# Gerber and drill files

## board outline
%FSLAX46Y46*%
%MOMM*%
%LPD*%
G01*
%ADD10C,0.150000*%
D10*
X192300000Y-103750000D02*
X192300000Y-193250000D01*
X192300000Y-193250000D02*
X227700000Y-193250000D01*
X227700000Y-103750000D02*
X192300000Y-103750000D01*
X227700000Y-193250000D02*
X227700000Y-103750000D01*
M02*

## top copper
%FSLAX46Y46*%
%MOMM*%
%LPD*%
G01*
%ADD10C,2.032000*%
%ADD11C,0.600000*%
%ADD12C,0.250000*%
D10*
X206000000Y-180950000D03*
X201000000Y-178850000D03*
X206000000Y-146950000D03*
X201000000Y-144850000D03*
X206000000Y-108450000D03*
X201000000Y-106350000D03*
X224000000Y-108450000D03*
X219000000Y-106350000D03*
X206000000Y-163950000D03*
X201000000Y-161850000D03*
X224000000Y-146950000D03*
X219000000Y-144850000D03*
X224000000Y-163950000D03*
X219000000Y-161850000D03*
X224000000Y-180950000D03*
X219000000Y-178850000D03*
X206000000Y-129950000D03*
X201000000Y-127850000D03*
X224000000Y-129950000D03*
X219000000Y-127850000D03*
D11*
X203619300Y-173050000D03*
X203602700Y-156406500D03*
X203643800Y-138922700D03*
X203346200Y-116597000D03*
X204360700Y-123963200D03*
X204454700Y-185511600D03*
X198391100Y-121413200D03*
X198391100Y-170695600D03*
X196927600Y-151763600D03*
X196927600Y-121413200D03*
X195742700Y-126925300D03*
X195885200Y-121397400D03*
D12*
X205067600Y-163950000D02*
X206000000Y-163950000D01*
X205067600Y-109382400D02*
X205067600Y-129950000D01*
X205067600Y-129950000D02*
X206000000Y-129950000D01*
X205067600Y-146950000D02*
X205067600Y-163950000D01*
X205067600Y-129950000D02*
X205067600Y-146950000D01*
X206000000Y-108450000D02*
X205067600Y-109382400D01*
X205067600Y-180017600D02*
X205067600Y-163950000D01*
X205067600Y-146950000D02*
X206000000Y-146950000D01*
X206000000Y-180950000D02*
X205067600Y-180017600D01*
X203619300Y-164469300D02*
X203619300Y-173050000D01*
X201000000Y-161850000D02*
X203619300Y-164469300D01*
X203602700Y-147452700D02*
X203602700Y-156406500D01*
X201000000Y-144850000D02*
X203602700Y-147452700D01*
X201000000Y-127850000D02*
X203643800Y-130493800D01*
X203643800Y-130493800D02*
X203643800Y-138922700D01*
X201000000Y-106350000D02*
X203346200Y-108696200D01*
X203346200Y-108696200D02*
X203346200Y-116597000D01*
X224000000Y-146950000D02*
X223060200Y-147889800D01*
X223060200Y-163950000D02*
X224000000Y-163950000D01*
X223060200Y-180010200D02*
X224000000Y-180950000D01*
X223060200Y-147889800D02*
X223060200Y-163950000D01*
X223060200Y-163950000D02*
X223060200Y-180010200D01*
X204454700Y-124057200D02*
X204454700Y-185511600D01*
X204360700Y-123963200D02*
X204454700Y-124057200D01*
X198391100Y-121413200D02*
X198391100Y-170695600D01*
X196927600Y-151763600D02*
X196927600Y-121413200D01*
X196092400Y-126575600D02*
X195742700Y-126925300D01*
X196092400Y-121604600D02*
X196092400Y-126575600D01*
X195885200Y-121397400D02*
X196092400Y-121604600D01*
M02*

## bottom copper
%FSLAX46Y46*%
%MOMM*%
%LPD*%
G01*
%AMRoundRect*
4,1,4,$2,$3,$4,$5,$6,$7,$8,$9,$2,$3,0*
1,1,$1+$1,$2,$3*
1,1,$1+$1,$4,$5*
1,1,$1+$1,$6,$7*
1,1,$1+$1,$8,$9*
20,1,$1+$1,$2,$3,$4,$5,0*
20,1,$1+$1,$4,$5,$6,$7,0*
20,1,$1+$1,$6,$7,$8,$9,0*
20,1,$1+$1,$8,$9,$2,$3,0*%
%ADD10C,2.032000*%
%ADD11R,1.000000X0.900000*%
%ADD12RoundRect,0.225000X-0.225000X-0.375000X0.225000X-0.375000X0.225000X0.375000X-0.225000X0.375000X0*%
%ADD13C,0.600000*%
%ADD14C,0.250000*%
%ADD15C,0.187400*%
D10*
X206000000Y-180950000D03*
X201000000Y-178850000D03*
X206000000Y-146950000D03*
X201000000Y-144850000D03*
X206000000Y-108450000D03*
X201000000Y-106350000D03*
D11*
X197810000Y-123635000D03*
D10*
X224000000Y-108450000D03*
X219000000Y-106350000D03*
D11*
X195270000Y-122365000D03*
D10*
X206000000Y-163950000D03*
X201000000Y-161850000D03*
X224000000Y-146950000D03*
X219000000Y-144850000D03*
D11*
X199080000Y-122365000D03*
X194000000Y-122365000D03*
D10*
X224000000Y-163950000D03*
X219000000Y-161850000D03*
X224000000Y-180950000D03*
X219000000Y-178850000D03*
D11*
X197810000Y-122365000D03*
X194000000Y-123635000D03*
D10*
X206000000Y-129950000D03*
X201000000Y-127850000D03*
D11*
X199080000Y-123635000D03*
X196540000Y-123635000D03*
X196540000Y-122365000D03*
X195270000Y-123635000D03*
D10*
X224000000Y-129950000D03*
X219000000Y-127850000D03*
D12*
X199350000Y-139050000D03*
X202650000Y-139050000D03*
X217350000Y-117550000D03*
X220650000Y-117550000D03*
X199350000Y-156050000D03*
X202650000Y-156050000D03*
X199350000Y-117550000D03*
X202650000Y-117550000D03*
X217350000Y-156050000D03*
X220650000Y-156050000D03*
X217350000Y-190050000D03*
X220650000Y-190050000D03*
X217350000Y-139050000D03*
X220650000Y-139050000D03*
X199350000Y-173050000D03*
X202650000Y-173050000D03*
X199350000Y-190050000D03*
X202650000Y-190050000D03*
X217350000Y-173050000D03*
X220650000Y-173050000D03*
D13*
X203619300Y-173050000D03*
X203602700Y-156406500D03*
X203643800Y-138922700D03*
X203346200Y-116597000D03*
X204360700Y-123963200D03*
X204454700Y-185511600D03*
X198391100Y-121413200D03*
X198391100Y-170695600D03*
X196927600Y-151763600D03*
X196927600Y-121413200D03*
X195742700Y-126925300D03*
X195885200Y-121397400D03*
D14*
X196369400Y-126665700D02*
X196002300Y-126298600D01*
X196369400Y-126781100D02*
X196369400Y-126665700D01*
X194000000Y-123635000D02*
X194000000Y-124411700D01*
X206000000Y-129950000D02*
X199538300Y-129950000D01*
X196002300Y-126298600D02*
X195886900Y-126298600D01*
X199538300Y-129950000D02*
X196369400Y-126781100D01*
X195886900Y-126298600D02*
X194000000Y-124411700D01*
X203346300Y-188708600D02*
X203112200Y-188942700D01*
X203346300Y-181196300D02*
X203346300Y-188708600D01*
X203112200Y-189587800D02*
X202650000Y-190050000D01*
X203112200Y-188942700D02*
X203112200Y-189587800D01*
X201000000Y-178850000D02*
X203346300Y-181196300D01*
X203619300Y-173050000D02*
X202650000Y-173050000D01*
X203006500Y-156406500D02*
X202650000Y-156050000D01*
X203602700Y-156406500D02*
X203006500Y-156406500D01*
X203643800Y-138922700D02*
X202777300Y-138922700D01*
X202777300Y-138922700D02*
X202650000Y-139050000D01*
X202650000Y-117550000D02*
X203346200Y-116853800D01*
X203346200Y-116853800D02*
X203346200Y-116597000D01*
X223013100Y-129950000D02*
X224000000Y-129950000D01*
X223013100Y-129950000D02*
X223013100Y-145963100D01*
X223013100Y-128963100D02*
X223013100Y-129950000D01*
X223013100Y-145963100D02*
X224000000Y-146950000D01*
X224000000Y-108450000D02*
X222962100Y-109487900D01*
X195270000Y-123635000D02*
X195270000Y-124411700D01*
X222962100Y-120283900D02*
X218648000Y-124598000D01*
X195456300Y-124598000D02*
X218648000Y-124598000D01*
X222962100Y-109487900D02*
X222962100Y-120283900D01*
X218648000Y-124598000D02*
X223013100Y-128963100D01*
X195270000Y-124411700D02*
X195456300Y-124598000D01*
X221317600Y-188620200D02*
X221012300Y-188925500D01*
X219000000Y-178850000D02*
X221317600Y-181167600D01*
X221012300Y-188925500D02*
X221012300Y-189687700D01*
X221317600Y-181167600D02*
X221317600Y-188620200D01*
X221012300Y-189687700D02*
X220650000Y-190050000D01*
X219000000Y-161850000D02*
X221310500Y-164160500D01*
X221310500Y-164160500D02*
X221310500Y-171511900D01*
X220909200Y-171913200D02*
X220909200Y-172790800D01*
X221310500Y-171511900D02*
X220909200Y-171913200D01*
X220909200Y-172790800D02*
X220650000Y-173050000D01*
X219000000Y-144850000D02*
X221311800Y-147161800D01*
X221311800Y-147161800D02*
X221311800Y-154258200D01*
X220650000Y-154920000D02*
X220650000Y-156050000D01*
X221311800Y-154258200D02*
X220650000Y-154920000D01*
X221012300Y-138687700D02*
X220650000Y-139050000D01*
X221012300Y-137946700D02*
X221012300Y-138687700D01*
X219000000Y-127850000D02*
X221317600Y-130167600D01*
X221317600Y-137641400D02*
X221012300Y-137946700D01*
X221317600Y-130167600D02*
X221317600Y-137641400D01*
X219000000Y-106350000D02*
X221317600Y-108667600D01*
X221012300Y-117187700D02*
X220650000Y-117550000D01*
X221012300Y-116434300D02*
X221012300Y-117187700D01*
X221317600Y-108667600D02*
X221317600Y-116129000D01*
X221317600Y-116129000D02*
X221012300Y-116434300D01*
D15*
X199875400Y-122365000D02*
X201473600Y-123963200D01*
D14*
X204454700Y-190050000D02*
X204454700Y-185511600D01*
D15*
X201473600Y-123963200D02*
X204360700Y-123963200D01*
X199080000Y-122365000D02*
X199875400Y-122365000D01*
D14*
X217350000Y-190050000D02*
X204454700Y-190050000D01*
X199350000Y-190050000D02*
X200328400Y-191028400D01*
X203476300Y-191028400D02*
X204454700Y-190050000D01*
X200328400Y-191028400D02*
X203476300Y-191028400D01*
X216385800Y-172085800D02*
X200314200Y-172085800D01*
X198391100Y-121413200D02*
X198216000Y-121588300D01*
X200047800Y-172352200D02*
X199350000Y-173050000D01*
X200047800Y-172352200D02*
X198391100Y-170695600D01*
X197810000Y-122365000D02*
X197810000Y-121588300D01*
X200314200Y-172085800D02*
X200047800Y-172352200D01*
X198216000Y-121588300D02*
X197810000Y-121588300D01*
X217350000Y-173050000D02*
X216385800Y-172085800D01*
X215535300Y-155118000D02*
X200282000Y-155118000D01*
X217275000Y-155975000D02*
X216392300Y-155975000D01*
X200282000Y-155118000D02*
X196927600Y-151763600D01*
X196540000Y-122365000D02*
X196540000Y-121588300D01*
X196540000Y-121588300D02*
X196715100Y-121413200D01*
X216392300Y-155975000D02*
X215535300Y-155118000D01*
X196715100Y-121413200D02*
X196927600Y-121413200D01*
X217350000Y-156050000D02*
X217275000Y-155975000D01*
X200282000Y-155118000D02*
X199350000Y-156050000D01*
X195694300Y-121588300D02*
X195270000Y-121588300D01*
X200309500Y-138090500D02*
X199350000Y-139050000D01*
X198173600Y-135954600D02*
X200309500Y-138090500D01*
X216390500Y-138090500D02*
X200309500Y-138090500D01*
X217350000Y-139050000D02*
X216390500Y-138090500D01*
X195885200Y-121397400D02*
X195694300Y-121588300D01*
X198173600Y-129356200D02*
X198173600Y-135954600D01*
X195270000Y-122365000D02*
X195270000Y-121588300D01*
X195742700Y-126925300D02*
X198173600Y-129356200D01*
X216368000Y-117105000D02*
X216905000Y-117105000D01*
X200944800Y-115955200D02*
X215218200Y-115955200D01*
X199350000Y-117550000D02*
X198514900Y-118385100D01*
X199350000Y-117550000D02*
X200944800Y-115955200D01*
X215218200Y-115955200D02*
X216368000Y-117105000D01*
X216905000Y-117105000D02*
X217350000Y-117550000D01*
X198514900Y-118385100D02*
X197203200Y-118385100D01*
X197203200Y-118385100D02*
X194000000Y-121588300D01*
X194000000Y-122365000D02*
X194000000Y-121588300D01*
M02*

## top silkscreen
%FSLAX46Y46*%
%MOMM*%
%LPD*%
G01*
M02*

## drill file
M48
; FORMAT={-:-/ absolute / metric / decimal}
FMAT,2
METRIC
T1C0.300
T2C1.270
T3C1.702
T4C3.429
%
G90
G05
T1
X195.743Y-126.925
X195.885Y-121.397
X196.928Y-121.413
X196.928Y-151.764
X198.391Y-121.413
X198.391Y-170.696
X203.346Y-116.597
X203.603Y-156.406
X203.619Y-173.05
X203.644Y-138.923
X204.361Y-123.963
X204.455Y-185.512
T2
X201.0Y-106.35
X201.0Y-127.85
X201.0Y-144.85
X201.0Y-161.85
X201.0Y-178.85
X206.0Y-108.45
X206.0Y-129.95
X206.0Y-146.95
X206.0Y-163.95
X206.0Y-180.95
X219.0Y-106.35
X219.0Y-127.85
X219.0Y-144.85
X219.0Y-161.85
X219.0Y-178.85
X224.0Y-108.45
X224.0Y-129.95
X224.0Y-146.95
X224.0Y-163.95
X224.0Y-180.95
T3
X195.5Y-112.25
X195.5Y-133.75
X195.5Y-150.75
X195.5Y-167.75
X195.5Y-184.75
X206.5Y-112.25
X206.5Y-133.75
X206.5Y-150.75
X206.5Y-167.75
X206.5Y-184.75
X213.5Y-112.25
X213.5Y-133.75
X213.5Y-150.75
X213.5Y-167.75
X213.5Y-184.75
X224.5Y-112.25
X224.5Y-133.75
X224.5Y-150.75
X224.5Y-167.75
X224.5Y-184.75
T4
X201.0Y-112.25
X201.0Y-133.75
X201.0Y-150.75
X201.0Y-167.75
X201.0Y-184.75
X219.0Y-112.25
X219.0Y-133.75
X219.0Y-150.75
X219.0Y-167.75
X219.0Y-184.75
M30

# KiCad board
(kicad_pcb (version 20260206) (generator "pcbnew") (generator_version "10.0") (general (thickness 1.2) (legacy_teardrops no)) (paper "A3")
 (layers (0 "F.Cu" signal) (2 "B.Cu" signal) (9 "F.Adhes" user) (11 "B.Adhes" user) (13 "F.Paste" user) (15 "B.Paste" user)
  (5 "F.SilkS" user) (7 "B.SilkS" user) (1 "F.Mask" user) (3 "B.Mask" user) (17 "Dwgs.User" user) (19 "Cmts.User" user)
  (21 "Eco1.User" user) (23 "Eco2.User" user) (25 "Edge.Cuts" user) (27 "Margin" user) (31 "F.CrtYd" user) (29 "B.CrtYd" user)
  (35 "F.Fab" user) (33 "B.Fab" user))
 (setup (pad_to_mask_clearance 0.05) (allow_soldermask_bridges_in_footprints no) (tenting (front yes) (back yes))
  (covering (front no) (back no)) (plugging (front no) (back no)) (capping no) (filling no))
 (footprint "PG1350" (layer "F.Cu") (at 201 184.75)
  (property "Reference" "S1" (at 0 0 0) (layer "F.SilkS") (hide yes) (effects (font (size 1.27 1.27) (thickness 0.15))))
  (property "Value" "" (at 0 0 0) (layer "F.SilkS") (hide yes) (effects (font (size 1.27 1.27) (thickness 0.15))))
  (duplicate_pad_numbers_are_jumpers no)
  (pad "" np_thru_hole circle (at -5.5 0) (size 1.7018 1.7018) (drill 1.7018) (layers "*.Cu" "*.Mask"))
  (pad "" np_thru_hole circle (at 0 0) (size 3.429 3.429) (drill 3.429) (layers "*.Cu" "*.Mask"))
  (pad "" np_thru_hole circle (at 5.5 0) (size 1.7018 1.7018) (drill 1.7018) (layers "*.Cu" "*.Mask"))
  (pad "1" thru_hole circle (at 5 -3.8) (size 2.032 2.032) (drill 1.27) (layers "*.Cu" "*.Mask") (remove_unused_layers no) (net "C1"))
  (pad "2" thru_hole circle (at 0 -5.9) (size 2.032 2.032) (drill 1.27) (layers "*.Cu" "*.Mask") (remove_unused_layers no) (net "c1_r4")))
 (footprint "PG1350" (layer "F.Cu") (at 201 150.75)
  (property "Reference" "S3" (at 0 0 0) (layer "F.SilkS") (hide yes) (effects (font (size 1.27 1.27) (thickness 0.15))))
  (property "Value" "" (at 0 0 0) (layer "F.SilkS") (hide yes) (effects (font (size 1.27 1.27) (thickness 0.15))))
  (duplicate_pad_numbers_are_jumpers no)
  (pad "" np_thru_hole circle (at -5.5 0) (size 1.7018 1.7018) (drill 1.7018) (layers "*.Cu" "*.Mask"))
  (pad "" np_thru_hole circle (at 0 0) (size 3.429 3.429) (drill 3.429) (layers "*.Cu" "*.Mask"))
  (pad "" np_thru_hole circle (at 5.5 0) (size 1.7018 1.7018) (drill 1.7018) (layers "*.Cu" "*.Mask"))
  (pad "1" thru_hole circle (at 5 -3.8) (size 2.032 2.032) (drill 1.27) (layers "*.Cu" "*.Mask") (remove_unused_layers no) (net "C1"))
  (pad "2" thru_hole circle (at 0 -5.9) (size 2.032 2.032) (drill 1.27) (layers "*.Cu" "*.Mask") (remove_unused_layers no) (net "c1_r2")))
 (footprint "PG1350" (layer "F.Cu") (at 201 112.25)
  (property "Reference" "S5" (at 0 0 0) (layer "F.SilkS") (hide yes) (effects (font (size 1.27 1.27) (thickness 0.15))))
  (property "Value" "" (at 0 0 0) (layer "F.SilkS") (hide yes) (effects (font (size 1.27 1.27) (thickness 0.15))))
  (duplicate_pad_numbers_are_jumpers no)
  (pad "" np_thru_hole circle (at -5.5 0) (size 1.7018 1.7018) (drill 1.7018) (layers "*.Cu" "*.Mask"))
  (pad "" np_thru_hole circle (at 0 0) (size 3.429 3.429) (drill 3.429) (layers "*.Cu" "*.Mask"))
  (pad "" np_thru_hole circle (at 5.5 0) (size 1.7018 1.7018) (drill 1.7018) (layers "*.Cu" "*.Mask"))
  (pad "1" thru_hole circle (at 5 -3.8) (size 2.032 2.032) (drill 1.27) (layers "*.Cu" "*.Mask") (remove_unused_layers no) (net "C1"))
  (pad "2" thru_hole circle (at 0 -5.9) (size 2.032 2.032) (drill 1.27) (layers "*.Cu" "*.Mask") (remove_unused_layers no) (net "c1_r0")))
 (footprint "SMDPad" (layer "F.Cu") (at 197.81 123.635)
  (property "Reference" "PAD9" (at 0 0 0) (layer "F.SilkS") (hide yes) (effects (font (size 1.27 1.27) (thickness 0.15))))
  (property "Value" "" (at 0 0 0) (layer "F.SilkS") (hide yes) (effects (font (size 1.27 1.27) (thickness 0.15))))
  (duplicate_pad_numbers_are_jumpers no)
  (pad "1" smd rect (at 0 0) (size 1 0.9) (layers "B.Cu" "B.Mask" "B.Paste") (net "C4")))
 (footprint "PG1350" (layer "F.Cu") (at 219 112.25)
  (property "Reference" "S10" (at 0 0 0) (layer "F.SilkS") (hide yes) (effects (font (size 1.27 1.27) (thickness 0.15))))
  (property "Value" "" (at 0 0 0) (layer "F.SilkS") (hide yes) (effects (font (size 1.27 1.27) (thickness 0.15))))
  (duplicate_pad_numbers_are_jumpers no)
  (pad "" np_thru_hole circle (at -5.5 0) (size 1.7018 1.7018) (drill 1.7018) (layers "*.Cu" "*.Mask"))
  (pad "" np_thru_hole circle (at 0 0) (size 3.429 3.429) (drill 3.429) (layers "*.Cu" "*.Mask"))
  (pad "" np_thru_hole circle (at 5.5 0) (size 1.7018 1.7018) (drill 1.7018) (layers "*.Cu" "*.Mask"))
  (pad "1" thru_hole circle (at 5 -3.8) (size 2.032 2.032) (drill 1.27) (layers "*.Cu" "*.Mask") (remove_unused_layers no) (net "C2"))
  (pad "2" thru_hole circle (at 0 -5.9) (size 2.032 2.032) (drill 1.27) (layers "*.Cu" "*.Mask") (remove_unused_layers no) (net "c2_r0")))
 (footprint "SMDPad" (layer "F.Cu") (at 195.27 122.365)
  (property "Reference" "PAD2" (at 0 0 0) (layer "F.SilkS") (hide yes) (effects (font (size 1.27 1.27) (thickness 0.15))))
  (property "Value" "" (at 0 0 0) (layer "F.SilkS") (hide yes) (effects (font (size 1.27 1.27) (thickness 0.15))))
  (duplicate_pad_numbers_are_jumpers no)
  (pad "1" smd rect (at 0 0) (size 1 0.9) (layers "B.Cu" "B.Mask" "B.Paste") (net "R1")))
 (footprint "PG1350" (layer "F.Cu") (at 201 167.75)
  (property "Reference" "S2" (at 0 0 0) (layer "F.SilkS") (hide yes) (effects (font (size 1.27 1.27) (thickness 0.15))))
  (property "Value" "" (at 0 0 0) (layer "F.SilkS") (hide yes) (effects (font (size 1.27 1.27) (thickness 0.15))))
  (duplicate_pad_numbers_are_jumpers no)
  (pad "" np_thru_hole circle (at -5.5 0) (size 1.7018 1.7018) (drill 1.7018) (layers "*.Cu" "*.Mask"))
  (pad "" np_thru_hole circle (at 0 0) (size 3.429 3.429) (drill 3.429) (layers "*.Cu" "*.Mask"))
  (pad "" np_thru_hole circle (at 5.5 0) (size 1.7018 1.7018) (drill 1.7018) (layers "*.Cu" "*.Mask"))
  (pad "1" thru_hole circle (at 5 -3.8) (size 2.032 2.032) (drill 1.27) (layers "*.Cu" "*.Mask") (remove_unused_layers no) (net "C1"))
  (pad "2" thru_hole circle (at 0 -5.9) (size 2.032 2.032) (drill 1.27) (layers "*.Cu" "*.Mask") (remove_unused_layers no) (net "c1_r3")))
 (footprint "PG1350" (layer "F.Cu") (at 219 150.75)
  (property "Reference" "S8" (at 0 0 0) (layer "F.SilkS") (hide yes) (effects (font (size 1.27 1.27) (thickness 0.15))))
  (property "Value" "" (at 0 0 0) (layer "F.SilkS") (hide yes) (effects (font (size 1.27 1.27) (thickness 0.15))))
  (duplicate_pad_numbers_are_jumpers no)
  (pad "" np_thru_hole circle (at -5.5 0) (size 1.7018 1.7018) (drill 1.7018) (layers "*.Cu" "*.Mask"))
  (pad "" np_thru_hole circle (at 0 0) (size 3.429 3.429) (drill 3.429) (layers "*.Cu" "*.Mask"))
  (pad "" np_thru_hole circle (at 5.5 0) (size 1.7018 1.7018) (drill 1.7018) (layers "*.Cu" "*.Mask"))
  (pad "1" thru_hole circle (at 5 -3.8) (size 2.032 2.032) (drill 1.27) (layers "*.Cu" "*.Mask") (remove_unused_layers no) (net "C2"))
  (pad "2" thru_hole circle (at 0 -5.9) (size 2.032 2.032) (drill 1.27) (layers "*.Cu" "*.Mask") (remove_unused_layers no) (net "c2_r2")))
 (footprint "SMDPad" (layer "F.Cu") (at 199.08 122.365)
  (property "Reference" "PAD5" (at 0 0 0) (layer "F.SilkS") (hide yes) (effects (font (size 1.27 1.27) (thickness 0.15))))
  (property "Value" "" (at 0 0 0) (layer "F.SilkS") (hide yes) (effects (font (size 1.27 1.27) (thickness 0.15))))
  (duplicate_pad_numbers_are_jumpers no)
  (pad "1" smd rect (at 0 0) (size 1 0.9) (layers "B.Cu" "B.Mask" "B.Paste") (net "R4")))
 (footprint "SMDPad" (layer "F.Cu") (at 194 122.365)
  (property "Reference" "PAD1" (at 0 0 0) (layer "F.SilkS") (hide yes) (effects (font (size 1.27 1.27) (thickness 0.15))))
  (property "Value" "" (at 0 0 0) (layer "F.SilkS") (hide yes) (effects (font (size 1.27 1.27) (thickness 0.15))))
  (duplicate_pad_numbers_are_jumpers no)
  (pad "1" smd rect (at 0 0) (size 1 0.9) (layers "B.Cu" "B.Mask" "B.Paste") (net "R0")))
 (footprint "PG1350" (layer "F.Cu") (at 219 167.75)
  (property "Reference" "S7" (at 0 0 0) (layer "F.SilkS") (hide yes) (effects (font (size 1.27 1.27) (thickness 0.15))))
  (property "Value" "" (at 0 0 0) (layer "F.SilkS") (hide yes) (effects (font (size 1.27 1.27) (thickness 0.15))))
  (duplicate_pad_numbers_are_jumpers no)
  (pad "" np_thru_hole circle (at -5.5 0) (size 1.7018 1.7018) (drill 1.7018) (layers "*.Cu" "*.Mask"))
  (pad "" np_thru_hole circle (at 0 0) (size 3.429 3.429) (drill 3.429) (layers "*.Cu" "*.Mask"))
  (pad "" np_thru_hole circle (at 5.5 0) (size 1.7018 1.7018) (drill 1.7018) (layers "*.Cu" "*.Mask"))
  (pad "1" thru_hole circle (at 5 -3.8) (size 2.032 2.032) (drill 1.27) (layers "*.Cu" "*.Mask") (remove_unused_layers no) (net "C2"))
  (pad "2" thru_hole circle (at 0 -5.9) (size 2.032 2.032) (drill 1.27) (layers "*.Cu" "*.Mask") (remove_unused_layers no) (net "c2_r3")))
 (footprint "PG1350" (layer "F.Cu") (at 219 184.75)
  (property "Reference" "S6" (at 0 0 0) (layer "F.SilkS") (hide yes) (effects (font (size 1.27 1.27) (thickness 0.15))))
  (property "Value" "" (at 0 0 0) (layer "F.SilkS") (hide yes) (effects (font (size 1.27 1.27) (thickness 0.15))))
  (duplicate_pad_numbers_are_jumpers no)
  (pad "" np_thru_hole circle (at -5.5 0) (size 1.7018 1.7018) (drill 1.7018) (layers "*.Cu" "*.Mask"))
  (pad "" np_thru_hole circle (at 0 0) (size 3.429 3.429) (drill 3.429) (layers "*.Cu" "*.Mask"))
  (pad "" np_thru_hole circle (at 5.5 0) (size 1.7018 1.7018) (drill 1.7018) (layers "*.Cu" "*.Mask"))
  (pad "1" thru_hole circle (at 5 -3.8) (size 2.032 2.032) (drill 1.27) (layers "*.Cu" "*.Mask") (remove_unused_layers no) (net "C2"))
  (pad "2" thru_hole circle (at 0 -5.9) (size 2.032 2.032) (drill 1.27) (layers "*.Cu" "*.Mask") (remove_unused_layers no) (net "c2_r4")))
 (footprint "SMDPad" (layer "F.Cu") (at 197.81 122.365)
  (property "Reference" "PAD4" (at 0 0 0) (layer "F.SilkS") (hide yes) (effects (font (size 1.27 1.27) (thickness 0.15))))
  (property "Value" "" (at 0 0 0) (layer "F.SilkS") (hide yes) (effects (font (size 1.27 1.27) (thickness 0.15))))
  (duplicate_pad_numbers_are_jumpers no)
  (pad "1" smd rect (at 0 0) (size 1 0.9) (layers "B.Cu" "B.Mask" "B.Paste") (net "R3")))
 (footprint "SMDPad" (layer "F.Cu") (at 194 123.635)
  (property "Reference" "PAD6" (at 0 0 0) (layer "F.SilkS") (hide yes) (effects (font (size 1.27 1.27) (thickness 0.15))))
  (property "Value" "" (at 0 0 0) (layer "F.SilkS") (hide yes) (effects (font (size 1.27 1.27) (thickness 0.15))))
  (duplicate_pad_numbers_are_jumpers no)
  (pad "1" smd rect (at 0 0) (size 1 0.9) (layers "B.Cu" "B.Mask" "B.Paste") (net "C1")))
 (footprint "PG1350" (layer "F.Cu") (at 201 133.75)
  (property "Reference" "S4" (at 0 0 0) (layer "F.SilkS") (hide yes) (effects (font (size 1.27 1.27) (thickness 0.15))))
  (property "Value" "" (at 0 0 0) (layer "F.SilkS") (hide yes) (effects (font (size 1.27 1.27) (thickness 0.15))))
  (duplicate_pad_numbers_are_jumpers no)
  (pad "" np_thru_hole circle (at -5.5 0) (size 1.7018 1.7018) (drill 1.7018) (layers "*.Cu" "*.Mask"))
  (pad "" np_thru_hole circle (at 0 0) (size 3.429 3.429) (drill 3.429) (layers "*.Cu" "*.Mask"))
  (pad "" np_thru_hole circle (at 5.5 0) (size 1.7018 1.7018) (drill 1.7018) (layers "*.Cu" "*.Mask"))
  (pad "1" thru_hole circle (at 5 -3.8) (size 2.032 2.032) (drill 1.27) (layers "*.Cu" "*.Mask") (remove_unused_layers no) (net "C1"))
  (pad "2" thru_hole circle (at 0 -5.9) (size 2.032 2.032) (drill 1.27) (layers "*.Cu" "*.Mask") (remove_unused_layers no) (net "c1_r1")))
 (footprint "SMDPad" (layer "F.Cu") (at 199.08 123.635)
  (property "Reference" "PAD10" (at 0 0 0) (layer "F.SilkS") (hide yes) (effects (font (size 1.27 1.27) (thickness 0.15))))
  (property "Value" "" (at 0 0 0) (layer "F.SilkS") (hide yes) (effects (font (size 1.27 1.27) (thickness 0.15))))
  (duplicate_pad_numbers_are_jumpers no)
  (pad "1" smd rect (at 0 0) (size 1 0.9) (layers "B.Cu" "B.Mask" "B.Paste") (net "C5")))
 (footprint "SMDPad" (layer "F.Cu") (at 196.54 123.635)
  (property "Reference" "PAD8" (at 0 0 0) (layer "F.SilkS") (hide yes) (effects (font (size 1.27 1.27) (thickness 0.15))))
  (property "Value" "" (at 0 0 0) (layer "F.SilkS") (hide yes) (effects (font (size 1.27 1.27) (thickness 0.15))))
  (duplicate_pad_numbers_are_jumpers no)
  (pad "1" smd rect (at 0 0) (size 1 0.9) (layers "B.Cu" "B.Mask" "B.Paste") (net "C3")))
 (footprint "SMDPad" (layer "F.Cu") (at 196.54 122.365)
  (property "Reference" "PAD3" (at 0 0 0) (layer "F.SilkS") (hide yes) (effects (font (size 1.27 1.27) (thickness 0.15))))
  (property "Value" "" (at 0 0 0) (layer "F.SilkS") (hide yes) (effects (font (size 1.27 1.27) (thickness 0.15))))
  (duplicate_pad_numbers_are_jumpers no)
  (pad "1" smd rect (at 0 0) (size 1 0.9) (layers "B.Cu" "B.Mask" "B.Paste") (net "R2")))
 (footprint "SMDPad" (layer "F.Cu") (at 195.27 123.635)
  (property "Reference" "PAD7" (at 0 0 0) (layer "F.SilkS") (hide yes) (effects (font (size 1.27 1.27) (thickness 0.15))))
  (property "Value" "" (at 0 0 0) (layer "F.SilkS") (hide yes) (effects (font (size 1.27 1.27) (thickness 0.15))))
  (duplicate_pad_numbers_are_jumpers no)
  (pad "1" smd rect (at 0 0) (size 1 0.9) (layers "B.Cu" "B.Mask" "B.Paste") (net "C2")))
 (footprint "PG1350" (layer "F.Cu") (at 219 133.75)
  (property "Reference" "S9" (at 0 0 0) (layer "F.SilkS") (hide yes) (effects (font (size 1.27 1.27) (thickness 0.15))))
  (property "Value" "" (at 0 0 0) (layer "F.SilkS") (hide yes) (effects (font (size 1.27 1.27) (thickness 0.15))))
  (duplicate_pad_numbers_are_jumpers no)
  (pad "" np_thru_hole circle (at -5.5 0) (size 1.7018 1.7018) (drill 1.7018) (layers "*.Cu" "*.Mask"))
  (pad "" np_thru_hole circle (at 0 0) (size 3.429 3.429) (drill 3.429) (layers "*.Cu" "*.Mask"))
  (pad "" np_thru_hole circle (at 5.5 0) (size 1.7018 1.7018) (drill 1.7018) (layers "*.Cu" "*.Mask"))
  (pad "1" thru_hole circle (at 5 -3.8) (size 2.032 2.032) (drill 1.27) (layers "*.Cu" "*.Mask") (remove_unused_layers no) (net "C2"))
  (pad "2" thru_hole circle (at 0 -5.9) (size 2.032 2.032) (drill 1.27) (layers "*.Cu" "*.Mask") (remove_unused_layers no) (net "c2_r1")))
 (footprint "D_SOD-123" (layer "B.Cu") (at 201 139.05)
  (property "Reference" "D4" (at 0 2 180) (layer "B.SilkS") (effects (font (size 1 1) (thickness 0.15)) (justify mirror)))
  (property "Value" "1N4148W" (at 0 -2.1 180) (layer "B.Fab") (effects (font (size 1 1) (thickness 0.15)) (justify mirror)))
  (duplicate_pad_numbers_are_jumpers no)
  (pad "1" smd roundrect (at -1.65 0) (size 0.9 1.2) (layers "B.Cu" "B.Mask" "B.Paste") (roundrect_rratio 0.25) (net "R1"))
  (pad "2" smd roundrect (at 1.65 0) (size 0.9 1.2) (layers "B.Cu" "B.Mask" "B.Paste") (roundrect_rratio 0.25) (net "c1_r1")))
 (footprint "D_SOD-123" (layer "B.Cu") (at 219 117.55)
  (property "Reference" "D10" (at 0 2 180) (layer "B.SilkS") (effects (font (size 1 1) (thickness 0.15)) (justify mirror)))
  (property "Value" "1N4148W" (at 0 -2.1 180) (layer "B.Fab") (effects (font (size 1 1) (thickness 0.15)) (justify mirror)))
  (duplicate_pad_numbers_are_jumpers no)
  (pad "1" smd roundrect (at -1.65 0) (size 0.9 1.2) (layers "B.Cu" "B.Mask" "B.Paste") (roundrect_rratio 0.25) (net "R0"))
  (pad "2" smd roundrect (at 1.65 0) (size 0.9 1.2) (layers "B.Cu" "B.Mask" "B.Paste") (roundrect_rratio 0.25) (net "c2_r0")))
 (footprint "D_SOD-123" (layer "B.Cu") (at 201 156.05)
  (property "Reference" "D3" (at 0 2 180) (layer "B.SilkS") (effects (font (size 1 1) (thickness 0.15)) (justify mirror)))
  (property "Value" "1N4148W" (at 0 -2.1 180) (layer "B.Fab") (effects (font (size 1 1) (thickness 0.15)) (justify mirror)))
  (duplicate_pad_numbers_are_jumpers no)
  (pad "1" smd roundrect (at -1.65 0) (size 0.9 1.2) (layers "B.Cu" "B.Mask" "B.Paste") (roundrect_rratio 0.25) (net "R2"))
  (pad "2" smd roundrect (at 1.65 0) (size 0.9 1.2) (layers "B.Cu" "B.Mask" "B.Paste") (roundrect_rratio 0.25) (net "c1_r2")))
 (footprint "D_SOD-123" (layer "B.Cu") (at 201 117.55)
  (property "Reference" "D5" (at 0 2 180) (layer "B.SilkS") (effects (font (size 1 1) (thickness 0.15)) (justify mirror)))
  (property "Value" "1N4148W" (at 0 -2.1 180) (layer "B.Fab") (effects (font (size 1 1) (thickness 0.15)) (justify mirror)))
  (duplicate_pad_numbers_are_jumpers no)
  (pad "1" smd roundrect (at -1.65 0) (size 0.9 1.2) (layers "B.Cu" "B.Mask" "B.Paste") (roundrect_rratio 0.25) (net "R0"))
  (pad "2" smd roundrect (at 1.65 0) (size 0.9 1.2) (layers "B.Cu" "B.Mask" "B.Paste") (roundrect_rratio 0.25) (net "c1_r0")))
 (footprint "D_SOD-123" (layer "B.Cu") (at 219 156.05)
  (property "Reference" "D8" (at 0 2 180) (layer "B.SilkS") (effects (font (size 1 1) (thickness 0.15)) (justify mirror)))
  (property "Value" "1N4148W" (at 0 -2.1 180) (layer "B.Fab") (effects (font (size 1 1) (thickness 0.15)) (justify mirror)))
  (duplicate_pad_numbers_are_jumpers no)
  (pad "1" smd roundrect (at -1.65 0) (size 0.9 1.2) (layers "B.Cu" "B.Mask" "B.Paste") (roundrect_rratio 0.25) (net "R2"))
  (pad "2" smd roundrect (at 1.65 0) (size 0.9 1.2) (layers "B.Cu" "B.Mask" "B.Paste") (roundrect_rratio 0.25) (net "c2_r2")))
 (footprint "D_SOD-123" (layer "B.Cu") (at 219 190.05)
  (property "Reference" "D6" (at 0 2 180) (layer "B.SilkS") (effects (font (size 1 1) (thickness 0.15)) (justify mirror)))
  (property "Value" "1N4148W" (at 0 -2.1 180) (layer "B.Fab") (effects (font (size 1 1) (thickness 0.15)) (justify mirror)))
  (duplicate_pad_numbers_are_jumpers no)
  (pad "1" smd roundrect (at -1.65 0) (size 0.9 1.2) (layers "B.Cu" "B.Mask" "B.Paste") (roundrect_rratio 0.25) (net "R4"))
  (pad "2" smd roundrect (at 1.65 0) (size 0.9 1.2) (layers "B.Cu" "B.Mask" "B.Paste") (roundrect_rratio 0.25) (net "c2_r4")))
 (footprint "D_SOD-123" (layer "B.Cu") (at 219 139.05)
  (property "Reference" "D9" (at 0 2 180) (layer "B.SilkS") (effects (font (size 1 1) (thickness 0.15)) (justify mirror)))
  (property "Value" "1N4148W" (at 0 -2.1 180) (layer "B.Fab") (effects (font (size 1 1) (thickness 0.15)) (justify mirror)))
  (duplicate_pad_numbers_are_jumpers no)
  (pad "1" smd roundrect (at -1.65 0) (size 0.9 1.2) (layers "B.Cu" "B.Mask" "B.Paste") (roundrect_rratio 0.25) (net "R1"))
  (pad "2" smd roundrect (at 1.65 0) (size 0.9 1.2) (layers "B.Cu" "B.Mask" "B.Paste") (roundrect_rratio 0.25) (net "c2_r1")))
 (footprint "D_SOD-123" (layer "B.Cu") (at 201 173.05)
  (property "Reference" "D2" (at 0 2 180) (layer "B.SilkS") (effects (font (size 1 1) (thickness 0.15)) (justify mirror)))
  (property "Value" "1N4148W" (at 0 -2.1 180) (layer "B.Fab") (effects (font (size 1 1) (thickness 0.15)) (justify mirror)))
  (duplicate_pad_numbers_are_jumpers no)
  (pad "1" smd roundrect (at -1.65 0) (size 0.9 1.2) (layers "B.Cu" "B.Mask" "B.Paste") (roundrect_rratio 0.25) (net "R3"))
  (pad "2" smd roundrect (at 1.65 0) (size 0.9 1.2) (layers "B.Cu" "B.Mask" "B.Paste") (roundrect_rratio 0.25) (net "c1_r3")))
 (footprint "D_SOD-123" (layer "B.Cu") (at 201 190.05)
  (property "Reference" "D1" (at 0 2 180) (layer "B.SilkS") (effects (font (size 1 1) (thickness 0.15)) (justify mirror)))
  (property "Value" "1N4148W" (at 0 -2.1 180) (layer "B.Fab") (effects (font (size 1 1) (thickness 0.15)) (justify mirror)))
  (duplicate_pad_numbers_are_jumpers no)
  (pad "1" smd roundrect (at -1.65 0) (size 0.9 1.2) (layers "B.Cu" "B.Mask" "B.Paste") (roundrect_rratio 0.25) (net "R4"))
  (pad "2" smd roundrect (at 1.65 0) (size 0.9 1.2) (layers "B.Cu" "B.Mask" "B.Paste") (roundrect_rratio 0.25) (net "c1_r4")))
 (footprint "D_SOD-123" (layer "B.Cu") (at 219 173.05)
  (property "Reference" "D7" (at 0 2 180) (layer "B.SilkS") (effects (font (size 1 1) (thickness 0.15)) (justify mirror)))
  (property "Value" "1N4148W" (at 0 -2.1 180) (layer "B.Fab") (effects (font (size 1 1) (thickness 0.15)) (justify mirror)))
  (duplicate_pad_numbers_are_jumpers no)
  (pad "1" smd roundrect (at -1.65 0) (size 0.9 1.2) (layers "B.Cu" "B.Mask" "B.Paste") (roundrect_rratio 0.25) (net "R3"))
  (pad "2" smd roundrect (at 1.65 0) (size 0.9 1.2) (layers "B.Cu" "B.Mask" "B.Paste") (roundrect_rratio 0.25) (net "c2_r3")))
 (gr_line (start 192.3 103.75) (end 192.3 193.25) (stroke (width 0.15) (type solid)) (layer "Edge.Cuts"))
 (gr_line (start 192.3 193.25) (end 227.7 193.25) (stroke (width 0.15) (type solid)) (layer "Edge.Cuts"))
 (gr_line (start 227.7 103.75) (end 192.3 103.75) (stroke (width 0.15) (type solid)) (layer "Edge.Cuts"))
 (gr_line (start 227.7 193.25) (end 227.7 103.75) (stroke (width 0.15) (type solid)) (layer "Edge.Cuts"))
 (segment (start 205.0676 163.95) (end 206 163.95) (width 0.25) (layer "F.Cu") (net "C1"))
 (segment (start 205.0676 109.3824) (end 205.0676 129.95) (width 0.25) (layer "F.Cu") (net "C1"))
 (segment (start 205.0676 129.95) (end 206 129.95) (width 0.25) (layer "F.Cu") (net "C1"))
 (segment (start 205.0676 146.95) (end 205.0676 163.95) (width 0.25) (layer "F.Cu") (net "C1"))
 (segment (start 205.0676 129.95) (end 205.0676 146.95) (width 0.25) (layer "F.Cu") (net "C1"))
 (segment (start 206 108.45) (end 205.0676 109.3824) (width 0.25) (layer "F.Cu") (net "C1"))
 (segment (start 205.0676 180.0176) (end 205.0676 163.95) (width 0.25) (layer "F.Cu") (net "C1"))
 (segment (start 205.0676 146.95) (end 206 146.95) (width 0.25) (layer "F.Cu") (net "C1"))
 (segment (start 206 180.95) (end 205.0676 180.0176) (width 0.25) (layer "F.Cu") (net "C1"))
 (segment (start 196.3694 126.6657) (end 196.0023 126.2986) (width 0.25) (layer "B.Cu") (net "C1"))
 (segment (start 196.3694 126.7811) (end 196.3694 126.6657) (width 0.25) (layer "B.Cu") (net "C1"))
 (segment (start 194 123.635) (end 194 124.4117) (width 0.25) (layer "B.Cu") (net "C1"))
 (segment (start 206 129.95) (end 199.5383 129.95) (width 0.25) (layer "B.Cu") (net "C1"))
 (segment (start 196.0023 126.2986) (end 195.8869 126.2986) (width 0.25) (layer "B.Cu") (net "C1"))
 (segment (start 199.5383 129.95) (end 196.3694 126.7811) (width 0.25) (layer "B.Cu") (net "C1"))
 (segment (start 195.8869 126.2986) (end 194 124.4117) (width 0.25) (layer "B.Cu") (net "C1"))
 (segment (start 203.3463 188.7086) (end 203.1122 188.9427) (width 0.25) (layer "B.Cu") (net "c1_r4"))
 (segment (start 203.3463 181.1963) (end 203.3463 188.7086) (width 0.25) (layer "B.Cu") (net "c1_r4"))
 (segment (start 203.1122 189.5878) (end 202.65 190.05) (width 0.25) (layer "B.Cu") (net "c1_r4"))
 (segment (start 203.1122 188.9427) (end 203.1122 189.5878) (width 0.25) (layer "B.Cu") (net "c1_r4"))
 (segment (start 201 178.85) (end 203.3463 181.1963) (width 0.25) (layer "B.Cu") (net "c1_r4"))
 (segment (start 203.6193 164.4693) (end 203.6193 173.05) (width 0.25) (layer "F.Cu") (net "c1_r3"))
 (segment (start 201 161.85) (end 203.6193 164.4693) (width 0.25) (layer "F.Cu") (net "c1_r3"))
 (via (at 203.6193 173.05) (size 0.6) (drill 0.3) (layers "F.Cu" "B.Cu") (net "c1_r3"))
 (segment (start 203.6193 173.05) (end 202.65 173.05) (width 0.25) (layer "B.Cu") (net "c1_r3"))
 (segment (start 203.6027 147.4527) (end 203.6027 156.4065) (width 0.25) (layer "F.Cu") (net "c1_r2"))
 (segment (start 201 144.85) (end 203.6027 147.4527) (width 0.25) (layer "F.Cu") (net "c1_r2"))
 (via (at 203.6027 156.4065) (size 0.6) (drill 0.3) (layers "F.Cu" "B.Cu") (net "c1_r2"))
 (segment (start 203.0065 156.4065) (end 202.65 156.05) (width 0.25) (layer "B.Cu") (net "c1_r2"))
 (segment (start 203.6027 156.4065) (end 203.0065 156.4065) (width 0.25) (layer "B.Cu") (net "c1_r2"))
 (segment (start 201 127.85) (end 203.6438 130.4938) (width 0.25) (layer "F.Cu") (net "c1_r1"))
 (segment (start 203.6438 130.4938) (end 203.6438 138.9227) (width 0.25) (layer "F.Cu") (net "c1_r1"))
 (via (at 203.6438 138.9227) (size 0.6) (drill 0.3) (layers "F.Cu" "B.Cu") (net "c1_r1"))
 (segment (start 203.6438 138.9227) (end 202.7773 138.9227) (width 0.25) (layer "B.Cu") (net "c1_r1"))
 (segment (start 202.7773 138.9227) (end 202.65 139.05) (width 0.25) (layer "B.Cu") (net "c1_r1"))
 (segment (start 201 106.35) (end 203.3462 108.6962) (width 0.25) (layer "F.Cu") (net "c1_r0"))
 (segment (start 203.3462 108.6962) (end 203.3462 116.597) (width 0.25) (layer "F.Cu") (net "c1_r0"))
 (via (at 203.3462 116.597) (size 0.6) (drill 0.3) (layers "F.Cu" "B.Cu") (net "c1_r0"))
 (segment (start 202.65 117.55) (end 203.3462 116.8538) (width 0.25) (layer "B.Cu") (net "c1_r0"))
 (segment (start 203.3462 116.8538) (end 203.3462 116.597) (width 0.25) (layer "B.Cu") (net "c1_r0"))
 (segment (start 224 146.95) (end 223.0602 147.8898) (width 0.25) (layer "F.Cu") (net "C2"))
 (segment (start 223.0602 163.95) (end 224 163.95) (width 0.25) (layer "F.Cu") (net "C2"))
 (segment (start 223.0602 180.0102) (end 224 180.95) (width 0.25) (layer "F.Cu") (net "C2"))
 (segment (start 223.0602 147.8898) (end 223.0602 163.95) (width 0.25) (layer "F.Cu") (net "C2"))
 (segment (start 223.0602 163.95) (end 223.0602 180.0102) (width 0.25) (layer "F.Cu") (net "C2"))
 (segment (start 223.0131 129.95) (end 224 129.95) (width 0.25) (layer "B.Cu") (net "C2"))
 (segment (start 223.0131 129.95) (end 223.0131 145.9631) (width 0.25) (layer "B.Cu") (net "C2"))
 (segment (start 223.0131 128.9631) (end 223.0131 129.95) (width 0.25) (layer "B.Cu") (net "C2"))
 (segment (start 223.0131 145.9631) (end 224 146.95) (width 0.25) (layer "B.Cu") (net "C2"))
 (segment (start 224 108.45) (end 222.9621 109.4879) (width 0.25) (layer "B.Cu") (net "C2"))
 (segment (start 195.27 123.635) (end 195.27 124.4117) (width 0.25) (layer "B.Cu") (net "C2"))
 (segment (start 222.9621 120.2839) (end 218.648 124.598) (width 0.25) (layer "B.Cu") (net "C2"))
 (segment (start 195.4563 124.598) (end 218.648 124.598) (width 0.25) (layer "B.Cu") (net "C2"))
 (segment (start 222.9621 109.4879) (end 222.9621 120.2839) (width 0.25) (layer "B.Cu") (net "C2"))
 (segment (start 218.648 124.598) (end 223.0131 128.9631) (width 0.25) (layer "B.Cu") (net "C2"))
 (segment (start 195.27 124.4117) (end 195.4563 124.598) (width 0.25) (layer "B.Cu") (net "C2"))
 (segment (start 221.3176 188.6202) (end 221.0123 188.9255) (width 0.25) (layer "B.Cu") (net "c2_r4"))
 (segment (start 219 178.85) (end 221.3176 181.1676) (width 0.25) (layer "B.Cu") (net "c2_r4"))
 (segment (start 221.0123 188.9255) (end 221.0123 189.6877) (width 0.25) (layer "B.Cu") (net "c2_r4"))
 (segment (start 221.3176 181.1676) (end 221.3176 188.6202) (width 0.25) (layer "B.Cu") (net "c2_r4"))
 (segment (start 221.0123 189.6877) (end 220.65 190.05) (width 0.25) (layer "B.Cu") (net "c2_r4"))
 (segment (start 219 161.85) (end 221.3105 164.1605) (width 0.25) (layer "B.Cu") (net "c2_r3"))
 (segment (start 221.3105 164.1605) (end 221.3105 171.5119) (width 0.25) (layer "B.Cu") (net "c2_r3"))
 (segment (start 220.9092 171.9132) (end 220.9092 172.7908) (width 0.25) (layer "B.Cu") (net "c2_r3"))
 (segment (start 221.3105 171.5119) (end 220.9092 171.9132) (width 0.25) (layer "B.Cu") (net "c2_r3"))
 (segment (start 220.9092 172.7908) (end 220.65 173.05) (width 0.25) (layer "B.Cu") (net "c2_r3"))
 (segment (start 219 144.85) (end 221.3118 147.1618) (width 0.25) (layer "B.Cu") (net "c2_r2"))
 (segment (start 221.3118 147.1618) (end 221.3118 154.2582) (width 0.25) (layer "B.Cu") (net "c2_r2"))
 (segment (start 220.65 154.92) (end 220.65 156.05) (width 0.25) (layer "B.Cu") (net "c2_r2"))
 (segment (start 221.3118 154.2582) (end 220.65 154.92) (width 0.25) (layer "B.Cu") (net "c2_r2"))
 (segment (start 221.0123 138.6877) (end 220.65 139.05) (width 0.25) (layer "B.Cu") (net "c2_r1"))
 (segment (start 221.0123 137.9467) (end 221.0123 138.6877) (width 0.25) (layer "B.Cu") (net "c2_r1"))
 (segment (start 219 127.85) (end 221.3176 130.1676) (width 0.25) (layer "B.Cu") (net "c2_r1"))
 (segment (start 221.3176 137.6414) (end 221.0123 137.9467) (width 0.25) (layer "B.Cu") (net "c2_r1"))
 (segment (start 221.3176 130.1676) (end 221.3176 137.6414) (width 0.25) (layer "B.Cu") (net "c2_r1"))
 (segment (start 219 106.35) (end 221.3176 108.6676) (width 0.25) (layer "B.Cu") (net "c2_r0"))
 (segment (start 221.0123 117.1877) (end 220.65 117.55) (width 0.25) (layer "B.Cu") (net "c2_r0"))
 (segment (start 221.0123 116.4343) (end 221.0123 117.1877) (width 0.25) (layer "B.Cu") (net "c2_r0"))
 (segment (start 221.3176 108.6676) (end 221.3176 116.129) (width 0.25) (layer "B.Cu") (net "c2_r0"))
 (segment (start 221.3176 116.129) (end 221.0123 116.4343) (width 0.25) (layer "B.Cu") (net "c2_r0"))
 (segment (start 204.4547 124.0572) (end 204.4547 185.5116) (width 0.25) (layer "F.Cu") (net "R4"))
 (segment (start 204.3607 123.9632) (end 204.4547 124.0572) (width 0.25) (layer "F.Cu") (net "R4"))
 (via (at 204.3607 123.9632) (size 0.6) (drill 0.3) (layers "F.Cu" "B.Cu") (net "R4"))
 (via (at 204.4547 185.5116) (size 0.6) (drill 0.3) (layers "F.Cu" "B.Cu") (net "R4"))
 (segment (start 199.8754 122.365) (end 201.4736 123.9632) (width 0.1874) (layer "B.Cu") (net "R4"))
 (segment (start 204.4547 190.05) (end 204.4547 185.5116) (width 0.25) (layer "B.Cu") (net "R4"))
 (segment (start 201.4736 123.9632) (end 204.3607 123.9632) (width 0.1874) (layer "B.Cu") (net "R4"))
 (segment (start 199.08 122.365) (end 199.8754 122.365) (width 0.1874) (layer "B.Cu") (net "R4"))
 (segment (start 217.35 190.05) (end 204.4547 190.05) (width 0.25) (layer "B.Cu") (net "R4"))
 (segment (start 199.35 190.05) (end 200.3284 191.0284) (width 0.25) (layer "B.Cu") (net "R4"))
 (segment (start 203.4763 191.0284) (end 204.4547 190.05) (width 0.25) (layer "B.Cu") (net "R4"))
 (segment (start 200.3284 191.0284) (end 203.4763 191.0284) (width 0.25) (layer "B.Cu") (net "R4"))
 (segment (start 198.3911 121.4132) (end 198.3911 170.6956) (width 0.25) (layer "F.Cu") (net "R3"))
 (via (at 198.3911 121.4132) (size 0.6) (drill 0.3) (layers "F.Cu" "B.Cu") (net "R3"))
 (via (at 198.3911 170.6956) (size 0.6) (drill 0.3) (layers "F.Cu" "B.Cu") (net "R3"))
 (segment (start 216.3858 172.0858) (end 200.3142 172.0858) (width 0.25) (layer "B.Cu") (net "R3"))
 (segment (start 198.3911 121.4132) (end 198.216 121.5883) (width 0.25) (layer "B.Cu") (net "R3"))
 (segment (start 200.0478 172.3522) (end 199.35 173.05) (width 0.25) (layer "B.Cu") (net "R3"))
 (segment (start 200.0478 172.3522) (end 198.3911 170.6956) (width 0.25) (layer "B.Cu") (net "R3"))
 (segment (start 197.81 122.365) (end 197.81 121.5883) (width 0.25) (layer "B.Cu") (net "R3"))
 (segment (start 200.3142 172.0858) (end 200.0478 172.3522) (width 0.25) (layer "B.Cu") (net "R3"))
 (segment (start 198.216 121.5883) (end 197.81 121.5883) (width 0.25) (layer "B.Cu") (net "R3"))
 (segment (start 217.35 173.05) (end 216.3858 172.0858) (width 0.25) (layer "B.Cu") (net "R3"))
 (segment (start 196.9276 151.7636) (end 196.9276 121.4132) (width 0.25) (layer "F.Cu") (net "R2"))
 (via (at 196.9276 151.7636) (size 0.6) (drill 0.3) (layers "F.Cu" "B.Cu") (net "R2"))
 (via (at 196.9276 121.4132) (size 0.6) (drill 0.3) (layers "F.Cu" "B.Cu") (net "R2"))
 (segment (start 215.5353 155.118) (end 200.282 155.118) (width 0.25) (layer "B.Cu") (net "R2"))
 (segment (start 217.275 155.975) (end 216.3923 155.975) (width 0.25) (layer "B.Cu") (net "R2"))
 (segment (start 200.282 155.118) (end 196.9276 151.7636) (width 0.25) (layer "B.Cu") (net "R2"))
 (segment (start 196.54 122.365) (end 196.54 121.5883) (width 0.25) (layer "B.Cu") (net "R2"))
 (segment (start 196.54 121.5883) (end 196.7151 121.4132) (width 0.25) (layer "B.Cu") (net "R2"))
 (segment (start 216.3923 155.975) (end 215.5353 155.118) (width 0.25) (layer "B.Cu") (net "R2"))
 (segment (start 196.7151 121.4132) (end 196.9276 121.4132) (width 0.25) (layer "B.Cu") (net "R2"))
 (segment (start 217.35 156.05) (end 217.275 155.975) (width 0.25) (layer "B.Cu") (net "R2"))
 (segment (start 200.282 155.118) (end 199.35 156.05) (width 0.25) (layer "B.Cu") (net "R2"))
 (segment (start 196.0924 126.5756) (end 195.7427 126.9253) (width 0.25) (layer "F.Cu") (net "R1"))
 (segment (start 196.0924 121.6046) (end 196.0924 126.5756) (width 0.25) (layer "F.Cu") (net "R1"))
 (segment (start 195.8852 121.3974) (end 196.0924 121.6046) (width 0.25) (layer "F.Cu") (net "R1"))
 (via (at 195.7427 126.9253) (size 0.6) (drill 0.3) (layers "F.Cu" "B.Cu") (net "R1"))
 (via (at 195.8852 121.3974) (size 0.6) (drill 0.3) (layers "F.Cu" "B.Cu") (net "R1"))
 (segment (start 195.6943 121.5883) (end 195.27 121.5883) (width 0.25) (layer "B.Cu") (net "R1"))
 (segment (start 200.3095 138.0905) (end 199.35 139.05) (width 0.25) (layer "B.Cu") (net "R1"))
 (segment (start 198.1736 135.9546) (end 200.3095 138.0905) (width 0.25) (layer "B.Cu") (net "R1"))
 (segment (start 216.3905 138.0905) (end 200.3095 138.0905) (width 0.25) (layer "B.Cu") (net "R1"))
 (segment (start 217.35 139.05) (end 216.3905 138.0905) (width 0.25) (layer "B.Cu") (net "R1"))
 (segment (start 195.8852 121.3974) (end 195.6943 121.5883) (width 0.25) (layer "B.Cu") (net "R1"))
 (segment (start 198.1736 129.3562) (end 198.1736 135.9546) (width 0.25) (layer "B.Cu") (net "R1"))
 (segment (start 195.27 122.365) (end 195.27 121.5883) (width 0.25) (layer "B.Cu") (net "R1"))
 (segment (start 195.7427 126.9253) (end 198.1736 129.3562) (width 0.25) (layer "B.Cu") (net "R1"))
 (segment (start 216.368 117.105) (end 216.905 117.105) (width 0.25) (layer "B.Cu") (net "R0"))
 (segment (start 200.9448 115.9552) (end 215.2182 115.9552) (width 0.25) (layer "B.Cu") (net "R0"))
 (segment (start 199.35 117.55) (end 198.5149 118.3851) (width 0.25) (layer "B.Cu") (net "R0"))
 (segment (start 199.35 117.55) (end 200.9448 115.9552) (width 0.25) (layer "B.Cu") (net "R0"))
 (segment (start 215.2182 115.9552) (end 216.368 117.105) (width 0.25) (layer "B.Cu") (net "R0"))
 (segment (start 216.905 117.105) (end 217.35 117.55) (width 0.25) (layer "B.Cu") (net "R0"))
 (segment (start 198.5149 118.3851) (end 197.2032 118.3851) (width 0.25) (layer "B.Cu") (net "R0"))
 (segment (start 197.2032 118.3851) (end 194 121.5883) (width 0.25) (layer "B.Cu") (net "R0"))
 (segment (start 194 122.365) (end 194 121.5883) (width 0.25) (layer "B.Cu") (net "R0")))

